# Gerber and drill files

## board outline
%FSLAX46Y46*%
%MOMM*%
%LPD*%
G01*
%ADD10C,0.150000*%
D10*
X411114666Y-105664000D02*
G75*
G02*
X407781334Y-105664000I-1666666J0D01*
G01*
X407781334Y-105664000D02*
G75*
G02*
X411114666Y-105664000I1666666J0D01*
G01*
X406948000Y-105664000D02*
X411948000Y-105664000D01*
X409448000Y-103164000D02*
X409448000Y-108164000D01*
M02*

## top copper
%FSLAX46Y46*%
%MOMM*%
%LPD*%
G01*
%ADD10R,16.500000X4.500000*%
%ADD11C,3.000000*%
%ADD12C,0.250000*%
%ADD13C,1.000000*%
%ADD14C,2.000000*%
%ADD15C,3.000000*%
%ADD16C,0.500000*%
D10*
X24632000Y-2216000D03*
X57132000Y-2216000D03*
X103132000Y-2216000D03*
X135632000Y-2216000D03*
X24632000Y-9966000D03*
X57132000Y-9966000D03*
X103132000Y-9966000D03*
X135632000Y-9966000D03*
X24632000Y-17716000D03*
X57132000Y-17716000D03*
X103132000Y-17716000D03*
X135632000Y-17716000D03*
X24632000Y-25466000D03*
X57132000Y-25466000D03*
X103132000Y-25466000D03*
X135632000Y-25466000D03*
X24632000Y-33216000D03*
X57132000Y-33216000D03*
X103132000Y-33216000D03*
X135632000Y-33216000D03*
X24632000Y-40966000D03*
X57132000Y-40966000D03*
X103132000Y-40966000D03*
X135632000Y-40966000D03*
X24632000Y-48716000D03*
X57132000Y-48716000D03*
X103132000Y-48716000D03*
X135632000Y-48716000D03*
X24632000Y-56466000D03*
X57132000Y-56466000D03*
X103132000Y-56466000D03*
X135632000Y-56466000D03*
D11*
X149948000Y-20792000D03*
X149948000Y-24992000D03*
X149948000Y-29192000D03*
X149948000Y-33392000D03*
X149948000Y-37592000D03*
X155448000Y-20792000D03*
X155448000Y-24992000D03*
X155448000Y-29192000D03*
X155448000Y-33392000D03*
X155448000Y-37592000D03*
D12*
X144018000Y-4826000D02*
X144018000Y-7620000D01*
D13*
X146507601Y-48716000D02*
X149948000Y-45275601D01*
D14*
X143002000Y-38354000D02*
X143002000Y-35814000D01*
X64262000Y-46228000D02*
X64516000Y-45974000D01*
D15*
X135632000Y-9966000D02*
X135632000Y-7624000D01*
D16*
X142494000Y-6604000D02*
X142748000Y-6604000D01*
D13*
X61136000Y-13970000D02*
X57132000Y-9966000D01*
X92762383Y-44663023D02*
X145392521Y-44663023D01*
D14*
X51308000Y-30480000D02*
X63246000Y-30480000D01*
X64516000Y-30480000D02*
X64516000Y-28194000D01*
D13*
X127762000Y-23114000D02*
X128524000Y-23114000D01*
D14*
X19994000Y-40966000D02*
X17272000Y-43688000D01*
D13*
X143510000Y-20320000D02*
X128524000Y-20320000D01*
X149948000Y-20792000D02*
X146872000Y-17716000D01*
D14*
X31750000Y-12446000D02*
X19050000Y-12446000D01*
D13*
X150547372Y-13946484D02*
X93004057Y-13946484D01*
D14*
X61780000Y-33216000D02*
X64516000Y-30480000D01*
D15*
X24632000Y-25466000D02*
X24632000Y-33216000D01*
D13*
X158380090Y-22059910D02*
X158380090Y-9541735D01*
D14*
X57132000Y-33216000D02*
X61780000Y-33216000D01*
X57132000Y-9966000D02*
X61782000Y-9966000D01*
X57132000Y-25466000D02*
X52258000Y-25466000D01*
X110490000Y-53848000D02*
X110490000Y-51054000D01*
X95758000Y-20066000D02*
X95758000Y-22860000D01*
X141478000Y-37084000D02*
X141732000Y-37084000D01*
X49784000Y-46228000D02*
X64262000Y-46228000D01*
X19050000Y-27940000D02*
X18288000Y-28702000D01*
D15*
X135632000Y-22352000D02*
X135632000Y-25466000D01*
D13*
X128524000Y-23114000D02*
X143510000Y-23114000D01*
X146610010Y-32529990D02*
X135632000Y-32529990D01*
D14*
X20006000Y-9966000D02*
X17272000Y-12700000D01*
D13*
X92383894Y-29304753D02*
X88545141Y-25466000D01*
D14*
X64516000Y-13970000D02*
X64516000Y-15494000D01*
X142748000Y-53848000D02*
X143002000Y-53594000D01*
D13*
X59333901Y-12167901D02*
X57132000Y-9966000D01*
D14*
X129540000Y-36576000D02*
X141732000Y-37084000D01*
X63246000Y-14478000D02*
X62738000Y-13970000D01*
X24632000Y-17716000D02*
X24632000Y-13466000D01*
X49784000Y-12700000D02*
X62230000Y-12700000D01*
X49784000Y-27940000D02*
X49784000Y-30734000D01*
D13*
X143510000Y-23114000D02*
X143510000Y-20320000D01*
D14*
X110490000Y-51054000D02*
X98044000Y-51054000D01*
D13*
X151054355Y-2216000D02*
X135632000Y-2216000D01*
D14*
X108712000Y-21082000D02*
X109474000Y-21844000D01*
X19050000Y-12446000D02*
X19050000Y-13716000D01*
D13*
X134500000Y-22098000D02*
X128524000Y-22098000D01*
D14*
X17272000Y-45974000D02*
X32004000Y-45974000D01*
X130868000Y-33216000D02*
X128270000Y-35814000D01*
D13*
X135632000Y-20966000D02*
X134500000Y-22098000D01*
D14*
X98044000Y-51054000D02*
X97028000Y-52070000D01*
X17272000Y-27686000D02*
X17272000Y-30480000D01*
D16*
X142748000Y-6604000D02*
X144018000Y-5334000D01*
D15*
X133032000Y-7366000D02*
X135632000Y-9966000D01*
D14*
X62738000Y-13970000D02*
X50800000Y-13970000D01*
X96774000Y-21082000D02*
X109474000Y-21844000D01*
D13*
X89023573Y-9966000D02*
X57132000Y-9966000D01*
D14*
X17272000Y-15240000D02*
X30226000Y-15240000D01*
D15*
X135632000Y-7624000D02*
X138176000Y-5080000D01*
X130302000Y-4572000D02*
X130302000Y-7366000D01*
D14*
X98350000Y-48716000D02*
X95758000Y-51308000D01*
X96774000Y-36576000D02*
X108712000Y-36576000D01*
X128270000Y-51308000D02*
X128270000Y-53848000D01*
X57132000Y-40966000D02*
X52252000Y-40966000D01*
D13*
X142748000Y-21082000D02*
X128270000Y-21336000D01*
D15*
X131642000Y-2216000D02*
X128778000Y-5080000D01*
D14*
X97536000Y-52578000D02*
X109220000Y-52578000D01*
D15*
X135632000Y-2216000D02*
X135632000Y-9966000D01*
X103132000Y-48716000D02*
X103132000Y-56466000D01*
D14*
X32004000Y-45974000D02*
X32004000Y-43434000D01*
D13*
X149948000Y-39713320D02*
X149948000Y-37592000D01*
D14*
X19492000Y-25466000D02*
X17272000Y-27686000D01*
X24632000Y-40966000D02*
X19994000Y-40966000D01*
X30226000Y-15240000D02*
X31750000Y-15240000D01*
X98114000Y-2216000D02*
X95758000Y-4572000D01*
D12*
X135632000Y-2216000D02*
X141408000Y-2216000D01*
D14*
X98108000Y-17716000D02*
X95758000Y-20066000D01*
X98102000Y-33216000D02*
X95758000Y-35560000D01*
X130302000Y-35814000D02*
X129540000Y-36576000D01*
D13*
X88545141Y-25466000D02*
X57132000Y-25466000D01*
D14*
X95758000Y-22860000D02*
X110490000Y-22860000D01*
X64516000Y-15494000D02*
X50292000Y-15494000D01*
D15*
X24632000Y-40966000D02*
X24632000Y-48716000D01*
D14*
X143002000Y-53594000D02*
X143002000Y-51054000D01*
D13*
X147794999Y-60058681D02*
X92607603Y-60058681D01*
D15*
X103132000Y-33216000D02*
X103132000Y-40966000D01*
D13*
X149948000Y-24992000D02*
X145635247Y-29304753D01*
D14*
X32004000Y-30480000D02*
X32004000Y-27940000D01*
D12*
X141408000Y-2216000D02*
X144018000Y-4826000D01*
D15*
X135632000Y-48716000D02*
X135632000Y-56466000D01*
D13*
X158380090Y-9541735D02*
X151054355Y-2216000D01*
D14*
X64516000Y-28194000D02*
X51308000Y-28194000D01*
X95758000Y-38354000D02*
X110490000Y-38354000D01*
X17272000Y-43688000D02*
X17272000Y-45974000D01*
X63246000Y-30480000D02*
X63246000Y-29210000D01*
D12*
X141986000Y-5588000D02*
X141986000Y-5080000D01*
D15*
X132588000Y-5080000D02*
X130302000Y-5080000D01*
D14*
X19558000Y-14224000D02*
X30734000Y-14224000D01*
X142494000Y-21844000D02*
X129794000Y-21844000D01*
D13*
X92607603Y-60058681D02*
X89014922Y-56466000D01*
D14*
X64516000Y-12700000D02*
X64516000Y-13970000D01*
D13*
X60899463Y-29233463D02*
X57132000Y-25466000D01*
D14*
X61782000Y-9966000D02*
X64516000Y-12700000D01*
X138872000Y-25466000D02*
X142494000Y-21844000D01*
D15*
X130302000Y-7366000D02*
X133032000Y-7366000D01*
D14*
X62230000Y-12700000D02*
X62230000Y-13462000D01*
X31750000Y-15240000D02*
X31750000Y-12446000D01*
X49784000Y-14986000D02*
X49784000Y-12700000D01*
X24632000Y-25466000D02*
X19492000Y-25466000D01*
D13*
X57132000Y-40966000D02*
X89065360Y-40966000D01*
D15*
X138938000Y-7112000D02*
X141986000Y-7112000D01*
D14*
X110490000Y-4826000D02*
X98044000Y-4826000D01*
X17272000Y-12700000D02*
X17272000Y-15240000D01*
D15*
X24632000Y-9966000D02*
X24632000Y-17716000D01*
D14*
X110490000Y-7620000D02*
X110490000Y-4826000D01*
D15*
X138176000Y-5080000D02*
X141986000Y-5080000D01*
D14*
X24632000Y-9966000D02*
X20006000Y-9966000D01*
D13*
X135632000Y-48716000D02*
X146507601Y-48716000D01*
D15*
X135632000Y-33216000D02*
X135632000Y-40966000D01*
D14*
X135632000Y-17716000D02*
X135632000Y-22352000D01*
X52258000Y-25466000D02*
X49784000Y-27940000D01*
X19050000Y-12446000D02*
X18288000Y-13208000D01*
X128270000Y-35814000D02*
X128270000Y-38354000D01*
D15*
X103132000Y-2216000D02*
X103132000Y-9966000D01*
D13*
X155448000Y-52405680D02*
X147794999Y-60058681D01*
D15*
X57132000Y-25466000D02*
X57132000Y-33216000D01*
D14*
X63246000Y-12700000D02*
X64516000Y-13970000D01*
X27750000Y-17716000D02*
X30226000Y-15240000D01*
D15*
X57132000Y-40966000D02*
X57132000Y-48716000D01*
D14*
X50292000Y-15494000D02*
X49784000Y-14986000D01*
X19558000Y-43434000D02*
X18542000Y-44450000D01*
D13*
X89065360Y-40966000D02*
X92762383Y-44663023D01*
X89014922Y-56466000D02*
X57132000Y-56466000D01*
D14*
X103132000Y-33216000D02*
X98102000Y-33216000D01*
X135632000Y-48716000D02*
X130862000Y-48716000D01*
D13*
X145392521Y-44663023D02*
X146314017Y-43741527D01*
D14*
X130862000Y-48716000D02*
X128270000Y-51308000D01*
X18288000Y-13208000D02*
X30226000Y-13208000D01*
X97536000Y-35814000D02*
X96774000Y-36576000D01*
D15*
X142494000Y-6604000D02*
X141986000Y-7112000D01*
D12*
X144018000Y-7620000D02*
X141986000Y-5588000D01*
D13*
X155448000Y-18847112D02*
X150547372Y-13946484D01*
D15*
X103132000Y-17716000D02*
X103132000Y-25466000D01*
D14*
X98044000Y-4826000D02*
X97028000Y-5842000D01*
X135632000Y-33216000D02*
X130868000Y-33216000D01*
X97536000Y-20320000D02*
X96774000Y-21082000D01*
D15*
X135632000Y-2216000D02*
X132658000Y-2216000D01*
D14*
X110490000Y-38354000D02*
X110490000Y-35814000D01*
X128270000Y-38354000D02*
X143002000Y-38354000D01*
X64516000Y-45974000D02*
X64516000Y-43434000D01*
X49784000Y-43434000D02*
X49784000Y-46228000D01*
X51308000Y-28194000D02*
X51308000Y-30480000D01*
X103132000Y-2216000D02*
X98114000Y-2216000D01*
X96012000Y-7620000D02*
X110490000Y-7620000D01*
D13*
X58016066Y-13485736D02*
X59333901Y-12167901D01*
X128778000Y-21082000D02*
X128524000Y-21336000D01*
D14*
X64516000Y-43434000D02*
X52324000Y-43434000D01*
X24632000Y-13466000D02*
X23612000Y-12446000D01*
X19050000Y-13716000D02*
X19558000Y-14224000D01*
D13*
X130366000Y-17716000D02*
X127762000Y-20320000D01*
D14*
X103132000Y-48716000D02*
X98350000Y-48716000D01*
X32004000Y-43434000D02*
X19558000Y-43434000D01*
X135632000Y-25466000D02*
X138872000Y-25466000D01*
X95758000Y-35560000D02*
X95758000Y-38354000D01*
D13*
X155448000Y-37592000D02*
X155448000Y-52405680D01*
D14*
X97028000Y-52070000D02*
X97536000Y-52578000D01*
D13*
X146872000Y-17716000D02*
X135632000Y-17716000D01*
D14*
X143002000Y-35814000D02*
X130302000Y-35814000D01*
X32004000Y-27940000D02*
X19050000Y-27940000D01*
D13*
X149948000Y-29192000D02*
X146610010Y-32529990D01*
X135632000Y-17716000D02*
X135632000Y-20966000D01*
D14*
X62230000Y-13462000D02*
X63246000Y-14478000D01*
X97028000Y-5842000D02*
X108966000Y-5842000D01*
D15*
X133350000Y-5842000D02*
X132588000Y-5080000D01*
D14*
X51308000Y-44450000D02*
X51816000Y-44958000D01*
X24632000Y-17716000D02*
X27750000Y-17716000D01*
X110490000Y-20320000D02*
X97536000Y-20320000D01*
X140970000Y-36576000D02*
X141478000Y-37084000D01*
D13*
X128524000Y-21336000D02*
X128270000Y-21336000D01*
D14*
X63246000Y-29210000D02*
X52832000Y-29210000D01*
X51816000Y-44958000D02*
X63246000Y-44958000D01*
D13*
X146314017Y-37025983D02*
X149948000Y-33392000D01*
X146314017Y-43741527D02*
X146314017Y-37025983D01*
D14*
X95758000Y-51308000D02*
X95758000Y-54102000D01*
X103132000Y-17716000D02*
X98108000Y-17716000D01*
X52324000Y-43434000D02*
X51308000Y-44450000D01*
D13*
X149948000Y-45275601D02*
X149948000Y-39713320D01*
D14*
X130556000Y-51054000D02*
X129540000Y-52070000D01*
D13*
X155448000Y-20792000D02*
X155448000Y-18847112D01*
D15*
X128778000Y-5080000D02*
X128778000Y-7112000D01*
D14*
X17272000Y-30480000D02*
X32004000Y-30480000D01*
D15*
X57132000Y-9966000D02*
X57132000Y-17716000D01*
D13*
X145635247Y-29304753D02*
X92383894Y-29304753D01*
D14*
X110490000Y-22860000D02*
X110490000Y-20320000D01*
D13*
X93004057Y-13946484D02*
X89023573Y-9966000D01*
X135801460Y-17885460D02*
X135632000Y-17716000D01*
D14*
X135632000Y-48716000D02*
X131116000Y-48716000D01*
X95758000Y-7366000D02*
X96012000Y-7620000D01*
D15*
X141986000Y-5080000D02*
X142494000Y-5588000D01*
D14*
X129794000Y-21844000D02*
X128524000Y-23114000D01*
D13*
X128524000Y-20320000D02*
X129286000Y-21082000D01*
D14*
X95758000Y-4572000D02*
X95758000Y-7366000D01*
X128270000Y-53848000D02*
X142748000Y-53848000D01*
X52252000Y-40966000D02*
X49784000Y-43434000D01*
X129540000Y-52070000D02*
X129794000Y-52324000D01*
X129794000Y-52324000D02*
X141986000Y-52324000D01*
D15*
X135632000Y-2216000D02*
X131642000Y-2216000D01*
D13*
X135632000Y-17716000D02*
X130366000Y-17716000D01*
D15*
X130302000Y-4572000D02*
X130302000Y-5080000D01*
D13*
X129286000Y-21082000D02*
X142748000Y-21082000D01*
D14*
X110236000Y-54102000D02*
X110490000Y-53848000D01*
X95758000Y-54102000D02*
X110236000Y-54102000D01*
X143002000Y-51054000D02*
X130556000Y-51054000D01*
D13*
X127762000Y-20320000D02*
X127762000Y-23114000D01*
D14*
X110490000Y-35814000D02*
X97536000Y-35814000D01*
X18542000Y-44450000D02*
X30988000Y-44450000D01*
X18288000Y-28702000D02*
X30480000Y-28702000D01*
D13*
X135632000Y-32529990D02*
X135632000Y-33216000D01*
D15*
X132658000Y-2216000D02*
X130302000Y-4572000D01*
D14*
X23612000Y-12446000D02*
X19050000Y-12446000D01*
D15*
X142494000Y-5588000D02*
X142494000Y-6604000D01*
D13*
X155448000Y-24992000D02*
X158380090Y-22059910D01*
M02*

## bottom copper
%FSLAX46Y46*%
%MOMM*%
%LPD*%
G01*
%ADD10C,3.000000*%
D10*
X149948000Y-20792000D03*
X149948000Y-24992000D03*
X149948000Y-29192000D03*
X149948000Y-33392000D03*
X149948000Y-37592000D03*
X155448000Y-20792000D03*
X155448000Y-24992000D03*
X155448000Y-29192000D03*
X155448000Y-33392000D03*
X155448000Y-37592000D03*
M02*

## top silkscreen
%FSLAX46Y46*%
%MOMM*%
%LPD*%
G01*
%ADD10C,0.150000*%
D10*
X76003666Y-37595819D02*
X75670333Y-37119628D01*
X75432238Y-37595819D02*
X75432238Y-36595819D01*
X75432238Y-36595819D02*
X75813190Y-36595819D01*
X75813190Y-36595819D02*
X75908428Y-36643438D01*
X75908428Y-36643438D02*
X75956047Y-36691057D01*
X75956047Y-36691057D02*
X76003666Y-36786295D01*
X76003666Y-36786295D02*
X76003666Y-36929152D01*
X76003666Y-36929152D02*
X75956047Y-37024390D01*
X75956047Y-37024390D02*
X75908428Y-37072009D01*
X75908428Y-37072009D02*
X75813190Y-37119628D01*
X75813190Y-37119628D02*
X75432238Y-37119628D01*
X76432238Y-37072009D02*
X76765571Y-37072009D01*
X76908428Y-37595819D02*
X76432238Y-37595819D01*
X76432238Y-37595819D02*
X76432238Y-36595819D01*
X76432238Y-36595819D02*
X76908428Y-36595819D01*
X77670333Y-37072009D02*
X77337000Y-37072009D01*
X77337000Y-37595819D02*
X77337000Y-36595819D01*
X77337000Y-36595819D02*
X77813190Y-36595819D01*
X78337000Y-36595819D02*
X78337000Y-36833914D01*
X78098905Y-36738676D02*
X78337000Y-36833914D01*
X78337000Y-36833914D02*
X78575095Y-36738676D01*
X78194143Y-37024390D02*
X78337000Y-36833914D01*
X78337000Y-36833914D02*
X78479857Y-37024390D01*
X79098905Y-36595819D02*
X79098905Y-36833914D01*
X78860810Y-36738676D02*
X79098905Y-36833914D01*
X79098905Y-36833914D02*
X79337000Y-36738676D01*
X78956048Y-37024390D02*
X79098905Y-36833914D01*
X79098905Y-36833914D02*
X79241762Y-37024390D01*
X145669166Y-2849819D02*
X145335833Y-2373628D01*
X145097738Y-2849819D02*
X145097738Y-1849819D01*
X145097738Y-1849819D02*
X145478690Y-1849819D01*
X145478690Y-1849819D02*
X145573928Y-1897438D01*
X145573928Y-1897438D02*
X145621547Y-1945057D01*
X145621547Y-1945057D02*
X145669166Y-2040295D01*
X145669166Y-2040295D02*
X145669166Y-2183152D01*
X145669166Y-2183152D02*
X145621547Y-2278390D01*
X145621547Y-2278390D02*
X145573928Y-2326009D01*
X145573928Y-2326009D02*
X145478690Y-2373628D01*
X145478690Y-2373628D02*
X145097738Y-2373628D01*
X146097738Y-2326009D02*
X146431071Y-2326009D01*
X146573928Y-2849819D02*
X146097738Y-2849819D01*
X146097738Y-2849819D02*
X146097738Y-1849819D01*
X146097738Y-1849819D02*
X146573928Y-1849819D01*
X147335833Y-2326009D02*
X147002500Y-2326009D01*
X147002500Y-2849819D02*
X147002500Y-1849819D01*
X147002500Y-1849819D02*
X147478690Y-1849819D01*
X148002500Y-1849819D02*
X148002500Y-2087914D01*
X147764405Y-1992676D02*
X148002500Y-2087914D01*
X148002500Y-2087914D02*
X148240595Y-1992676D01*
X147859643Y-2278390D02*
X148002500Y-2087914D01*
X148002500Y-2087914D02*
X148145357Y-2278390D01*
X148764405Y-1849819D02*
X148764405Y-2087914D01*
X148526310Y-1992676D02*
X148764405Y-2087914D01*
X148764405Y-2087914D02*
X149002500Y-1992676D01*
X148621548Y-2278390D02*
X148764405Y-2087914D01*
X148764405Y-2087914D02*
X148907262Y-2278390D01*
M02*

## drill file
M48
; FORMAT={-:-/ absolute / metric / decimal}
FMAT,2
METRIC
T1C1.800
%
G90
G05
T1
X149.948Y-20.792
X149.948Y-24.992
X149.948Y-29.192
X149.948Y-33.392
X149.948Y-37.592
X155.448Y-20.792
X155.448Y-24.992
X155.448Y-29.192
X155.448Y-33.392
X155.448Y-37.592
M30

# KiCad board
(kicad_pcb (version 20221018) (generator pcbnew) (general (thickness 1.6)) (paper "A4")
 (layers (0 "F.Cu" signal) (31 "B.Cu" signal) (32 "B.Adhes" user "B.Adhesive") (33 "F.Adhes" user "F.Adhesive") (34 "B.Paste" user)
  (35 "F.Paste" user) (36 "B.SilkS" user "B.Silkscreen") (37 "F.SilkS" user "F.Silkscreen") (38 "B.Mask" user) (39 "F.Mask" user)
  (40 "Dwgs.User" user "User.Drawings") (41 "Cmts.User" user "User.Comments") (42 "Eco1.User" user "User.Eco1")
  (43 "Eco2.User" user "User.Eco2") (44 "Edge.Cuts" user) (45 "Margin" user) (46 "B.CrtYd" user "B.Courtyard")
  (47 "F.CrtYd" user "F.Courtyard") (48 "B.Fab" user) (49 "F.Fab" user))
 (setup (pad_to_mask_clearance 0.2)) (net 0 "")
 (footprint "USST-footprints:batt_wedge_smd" (layer "F.Cu") (at 77.337 37.141)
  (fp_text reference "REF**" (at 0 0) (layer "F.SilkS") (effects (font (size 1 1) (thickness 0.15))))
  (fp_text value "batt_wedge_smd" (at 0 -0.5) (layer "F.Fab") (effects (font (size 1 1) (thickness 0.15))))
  (pad "1" smd rect (at -52.705 -34.925 90) (size 4.5 16.5) (layers "F.Cu" "F.Paste" "F.Mask"))
  (pad "1" smd rect (at -20.205 -34.925 90) (size 4.5 16.5) (layers "F.Cu" "F.Paste" "F.Mask"))
  (pad "1" smd rect (at 25.795 -34.925 90) (size 4.5 16.5) (layers "F.Cu" "F.Paste" "F.Mask"))
  (pad "1" smd rect (at 58.295 -34.925 90) (size 4.5 16.5) (layers "F.Cu" "F.Paste" "F.Mask"))
  (pad "2" smd rect (at -52.705 -27.175 90) (size 4.5 16.5) (layers "F.Cu" "F.Paste" "F.Mask"))
  (pad "2" smd rect (at -20.205 -27.175 90) (size 4.5 16.5) (layers "F.Cu" "F.Paste" "F.Mask"))
  (pad "2" smd rect (at 25.795 -27.175 90) (size 4.5 16.5) (layers "F.Cu" "F.Paste" "F.Mask"))
  (pad "2" smd rect (at 58.295 -27.175 90) (size 4.5 16.5) (layers "F.Cu" "F.Paste" "F.Mask"))
  (pad "3" smd rect (at -52.705 -19.425 90) (size 4.5 16.5) (layers "F.Cu" "F.Paste" "F.Mask"))
  (pad "3" smd rect (at -20.205 -19.425 90) (size 4.5 16.5) (layers "F.Cu" "F.Paste" "F.Mask"))
  (pad "3" smd rect (at 25.795 -19.425 90) (size 4.5 16.5) (layers "F.Cu" "F.Paste" "F.Mask"))
  (pad "3" smd rect (at 58.295 -19.425 90) (size 4.5 16.5) (layers "F.Cu" "F.Paste" "F.Mask"))
  (pad "4" smd rect (at -52.705 -11.675 90) (size 4.5 16.5) (layers "F.Cu" "F.Paste" "F.Mask"))
  (pad "4" smd rect (at -20.205 -11.675 90) (size 4.5 16.5) (layers "F.Cu" "F.Paste" "F.Mask"))
  (pad "4" smd rect (at 25.795 -11.675 90) (size 4.5 16.5) (layers "F.Cu" "F.Paste" "F.Mask"))
  (pad "4" smd rect (at 58.295 -11.675 90) (size 4.5 16.5) (layers "F.Cu" "F.Paste" "F.Mask"))
  (pad "5" smd rect (at -52.705 -3.925 90) (size 4.5 16.5) (layers "F.Cu" "F.Paste" "F.Mask"))
  (pad "5" smd rect (at -20.205 -3.925 90) (size 4.5 16.5) (layers "F.Cu" "F.Paste" "F.Mask"))
  (pad "5" smd rect (at 25.795 -3.925 90) (size 4.5 16.5) (layers "F.Cu" "F.Paste" "F.Mask"))
  (pad "5" smd rect (at 58.295 -3.925 90) (size 4.5 16.5) (layers "F.Cu" "F.Paste" "F.Mask"))
  (pad "6" smd rect (at -52.705 3.825 90) (size 4.5 16.5) (layers "F.Cu" "F.Paste" "F.Mask"))
  (pad "6" smd rect (at -20.205 3.825 90) (size 4.5 16.5) (layers "F.Cu" "F.Paste" "F.Mask"))
  (pad "6" smd rect (at 25.795 3.825 90) (size 4.5 16.5) (layers "F.Cu" "F.Paste" "F.Mask"))
  (pad "6" smd rect (at 58.295 3.825 90) (size 4.5 16.5) (layers "F.Cu" "F.Paste" "F.Mask"))
  (pad "7" smd rect (at -52.705 11.575 90) (size 4.5 16.5) (layers "F.Cu" "F.Paste" "F.Mask"))
  (pad "7" smd rect (at -20.205 11.575 90) (size 4.5 16.5) (layers "F.Cu" "F.Paste" "F.Mask"))
  (pad "7" smd rect (at 25.795 11.575 90) (size 4.5 16.5) (layers "F.Cu" "F.Paste" "F.Mask"))
  (pad "7" smd rect (at 58.295 11.575 90) (size 4.5 16.5) (layers "F.Cu" "F.Paste" "F.Mask"))
  (pad "8" smd rect (at -52.705 19.325 90) (size 4.5 16.5) (layers "F.Cu" "F.Paste" "F.Mask"))
  (pad "8" smd rect (at -20.205 19.325 90) (size 4.5 16.5) (layers "F.Cu" "F.Paste" "F.Mask"))
  (pad "8" smd rect (at 25.795 19.325 90) (size 4.5 16.5) (layers "F.Cu" "F.Paste" "F.Mask"))
  (pad "8" smd rect (at 58.295 19.325 90) (size 4.5 16.5) (layers "F.Cu" "F.Paste" "F.Mask")))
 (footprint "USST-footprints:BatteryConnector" (layer "F.Cu") (at 149.948 37.592)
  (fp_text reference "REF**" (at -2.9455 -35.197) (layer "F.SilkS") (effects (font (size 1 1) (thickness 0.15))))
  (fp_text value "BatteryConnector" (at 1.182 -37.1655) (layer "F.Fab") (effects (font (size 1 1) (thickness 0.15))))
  (pad "" np_thru_hole circle (at 0 -16.8) (size 3 3) (drill 1.8) (layers "*.Cu"))
  (pad "" np_thru_hole circle (at 0 -12.6) (size 3 3) (drill 1.8) (layers "*.Cu"))
  (pad "" np_thru_hole circle (at 0 -8.4) (size 3 3) (drill 1.8) (layers "*.Cu"))
  (pad "" np_thru_hole circle (at 0 -4.2) (size 3 3) (drill 1.8) (layers "*.Cu"))
  (pad "" np_thru_hole circle (at 0 0) (size 3 3) (drill 1.8) (layers "*.Cu"))
  (pad "" np_thru_hole circle (at 5.5 -16.8) (size 3 3) (drill 1.8) (layers "*.Cu"))
  (pad "" np_thru_hole circle (at 5.5 -12.6) (size 3 3) (drill 1.8) (layers "*.Cu"))
  (pad "" np_thru_hole circle (at 5.5 -8.4) (size 3 3) (drill 1.8) (layers "*.Cu"))
  (pad "" np_thru_hole circle (at 5.5 -4.2) (size 3 3) (drill 1.8) (layers "*.Cu"))
  (pad "" np_thru_hole circle (at 5.5 0) (size 3 3) (drill 1.8) (layers "*.Cu")))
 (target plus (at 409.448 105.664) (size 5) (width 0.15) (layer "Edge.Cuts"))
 (segment (start 144.018 4.826) (end 144.018 7.62) (width 0.25) (layer "F.Cu") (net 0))
 (segment (start 146.507601 48.716) (end 149.948 45.275601) (width 1) (layer "F.Cu") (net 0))
 (segment (start 143.002 38.354) (end 143.002 35.814) (width 2) (layer "F.Cu") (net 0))
 (segment (start 64.262 46.228) (end 64.516 45.974) (width 2) (layer "F.Cu") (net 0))
 (segment (start 135.632 9.966) (end 135.632 7.624) (width 3) (layer "F.Cu") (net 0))
 (segment (start 142.494 6.604) (end 142.748 6.604) (width 0.5) (layer "F.Cu") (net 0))
 (segment (start 61.136 13.97) (end 57.132 9.966) (width 1) (layer "F.Cu") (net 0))
 (segment (start 92.762383 44.663023) (end 145.392521 44.663023) (width 1) (layer "F.Cu") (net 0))
 (segment (start 51.308 30.48) (end 63.246 30.48) (width 2) (layer "F.Cu") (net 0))
 (segment (start 64.516 30.48) (end 64.516 28.194) (width 2) (layer "F.Cu") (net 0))
 (segment (start 127.762 23.114) (end 128.524 23.114) (width 1) (layer "F.Cu") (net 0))
 (segment (start 19.994 40.966) (end 17.272 43.688) (width 2) (layer "F.Cu") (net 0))
 (segment (start 143.51 20.32) (end 128.524 20.32) (width 1) (layer "F.Cu") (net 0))
 (segment (start 149.948 20.792) (end 146.872 17.716) (width 1) (layer "F.Cu") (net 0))
 (segment (start 31.75 12.446) (end 19.05 12.446) (width 2) (layer "F.Cu") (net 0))
 (segment (start 150.547372 13.946484) (end 93.004057 13.946484) (width 1) (layer "F.Cu") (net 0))
 (segment (start 61.78 33.216) (end 64.516 30.48) (width 2) (layer "F.Cu") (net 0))
 (segment (start 24.632 25.466) (end 24.632 33.216) (width 3) (layer "F.Cu") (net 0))
 (segment (start 158.38009 22.05991) (end 158.38009 9.541735) (width 1) (layer "F.Cu") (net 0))
 (segment (start 57.132 33.216) (end 61.78 33.216) (width 2) (layer "F.Cu") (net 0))
 (segment (start 57.132 9.966) (end 61.782 9.966) (width 2) (layer "F.Cu") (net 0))
 (segment (start 57.132 25.466) (end 52.258 25.466) (width 2) (layer "F.Cu") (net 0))
 (segment (start 110.49 53.848) (end 110.49 51.054) (width 2) (layer "F.Cu") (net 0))
 (segment (start 95.758 20.066) (end 95.758 22.86) (width 2) (layer "F.Cu") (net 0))
 (segment (start 141.478 37.084) (end 141.732 37.084) (width 2) (layer "F.Cu") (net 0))
 (segment (start 49.784 46.228) (end 64.262 46.228) (width 2) (layer "F.Cu") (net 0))
 (segment (start 19.05 27.94) (end 18.288 28.702) (width 2) (layer "F.Cu") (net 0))
 (segment (start 135.632 22.352) (end 135.632 25.466) (width 3) (layer "F.Cu") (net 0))
 (segment (start 128.524 23.114) (end 143.51 23.114) (width 1) (layer "F.Cu") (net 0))
 (segment (start 146.61001 32.52999) (end 135.632 32.52999) (width 1) (layer "F.Cu") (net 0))
 (segment (start 20.006 9.966) (end 17.272 12.7) (width 2) (layer "F.Cu") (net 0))
 (segment (start 92.383894 29.304753) (end 88.545141 25.466) (width 1) (layer "F.Cu") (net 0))
 (segment (start 64.516 13.97) (end 64.516 15.494) (width 2) (layer "F.Cu") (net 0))
 (segment (start 142.748 53.848) (end 143.002 53.594) (width 2) (layer "F.Cu") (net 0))
 (segment (start 59.333901 12.167901) (end 57.132 9.966) (width 1) (layer "F.Cu") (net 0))
 (segment (start 129.54 36.576) (end 141.732 37.084) (width 2) (layer "F.Cu") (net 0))
 (segment (start 63.246 14.478) (end 62.738 13.97) (width 2) (layer "F.Cu") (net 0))
 (segment (start 24.632 17.716) (end 24.632 13.466) (width 2) (layer "F.Cu") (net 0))
 (segment (start 49.784 12.7) (end 62.23 12.7) (width 2) (layer "F.Cu") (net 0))
 (segment (start 49.784 27.94) (end 49.784 30.734) (width 2) (layer "F.Cu") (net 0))
 (segment (start 143.51 23.114) (end 143.51 20.32) (width 1) (layer "F.Cu") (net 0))
 (segment (start 110.49 51.054) (end 98.044 51.054) (width 2) (layer "F.Cu") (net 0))
 (segment (start 151.054355 2.216) (end 135.632 2.216) (width 1) (layer "F.Cu") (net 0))
 (segment (start 108.712 21.082) (end 109.474 21.844) (width 2) (layer "F.Cu") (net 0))
 (segment (start 19.05 12.446) (end 19.05 13.716) (width 2) (layer "F.Cu") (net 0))
 (segment (start 134.5 22.098) (end 128.524 22.098) (width 1) (layer "F.Cu") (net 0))
 (segment (start 17.272 45.974) (end 32.004 45.974) (width 2) (layer "F.Cu") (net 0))
 (segment (start 130.868 33.216) (end 128.27 35.814) (width 2) (layer "F.Cu") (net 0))
 (segment (start 135.632 20.966) (end 134.5 22.098) (width 1) (layer "F.Cu") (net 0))
 (segment (start 98.044 51.054) (end 97.028 52.07) (width 2) (layer "F.Cu") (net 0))
 (segment (start 17.272 27.686) (end 17.272 30.48) (width 2) (layer "F.Cu") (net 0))
 (segment (start 142.748 6.604) (end 144.018 5.334) (width 0.5) (layer "F.Cu") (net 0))
 (segment (start 133.032 7.366) (end 135.632 9.966) (width 3) (layer "F.Cu") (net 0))
 (segment (start 62.738 13.97) (end 50.8 13.97) (width 2) (layer "F.Cu") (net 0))
 (segment (start 96.774 21.082) (end 109.474 21.844) (width 2) (layer "F.Cu") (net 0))
 (segment (start 89.023573 9.966) (end 57.132 9.966) (width 1) (layer "F.Cu") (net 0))
 (segment (start 17.272 15.24) (end 30.226 15.24) (width 2) (layer "F.Cu") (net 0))
 (segment (start 135.632 7.624) (end 138.176 5.08) (width 3) (layer "F.Cu") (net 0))
 (segment (start 130.302 4.572) (end 130.302 7.366) (width 3) (layer "F.Cu") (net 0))
 (segment (start 98.35 48.716) (end 95.758 51.308) (width 2) (layer "F.Cu") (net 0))
 (segment (start 96.774 36.576) (end 108.712 36.576) (width 2) (layer "F.Cu") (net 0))
 (segment (start 128.27 51.308) (end 128.27 53.848) (width 2) (layer "F.Cu") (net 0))
 (segment (start 57.132 40.966) (end 52.252 40.966) (width 2) (layer "F.Cu") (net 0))
 (segment (start 142.748 21.082) (end 128.27 21.336) (width 1) (layer "F.Cu") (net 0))
 (segment (start 131.642 2.216) (end 128.778 5.08) (width 3) (layer "F.Cu") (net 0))
 (segment (start 97.536 52.578) (end 109.22 52.578) (width 2) (layer "F.Cu") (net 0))
 (segment (start 135.632 2.216) (end 135.632 9.966) (width 3) (layer "F.Cu") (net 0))
 (segment (start 103.132 48.716) (end 103.132 56.466) (width 3) (layer "F.Cu") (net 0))
 (segment (start 32.004 45.974) (end 32.004 43.434) (width 2) (layer "F.Cu") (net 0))
 (segment (start 149.948 39.71332) (end 149.948 37.592) (width 1) (layer "F.Cu") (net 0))
 (segment (start 19.492 25.466) (end 17.272 27.686) (width 2) (layer "F.Cu") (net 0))
 (segment (start 24.632 40.966) (end 19.994 40.966) (width 2) (layer "F.Cu") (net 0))
 (segment (start 30.226 15.24) (end 31.75 15.24) (width 2) (layer "F.Cu") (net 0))
 (segment (start 98.114 2.216) (end 95.758 4.572) (width 2) (layer "F.Cu") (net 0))
 (segment (start 135.632 2.216) (end 141.408 2.216) (width 0.25) (layer "F.Cu") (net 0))
 (segment (start 98.108 17.716) (end 95.758 20.066) (width 2) (layer "F.Cu") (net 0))
 (segment (start 98.102 33.216) (end 95.758 35.56) (width 2) (layer "F.Cu") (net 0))
 (segment (start 130.302 35.814) (end 129.54 36.576) (width 2) (layer "F.Cu") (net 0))
 (segment (start 88.545141 25.466) (end 57.132 25.466) (width 1) (layer "F.Cu") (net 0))
 (segment (start 95.758 22.86) (end 110.49 22.86) (width 2) (layer "F.Cu") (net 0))
 (segment (start 64.516 15.494) (end 50.292 15.494) (width 2) (layer "F.Cu") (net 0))
 (segment (start 24.632 40.966) (end 24.632 48.716) (width 3) (layer "F.Cu") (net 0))
 (segment (start 143.002 53.594) (end 143.002 51.054) (width 2) (layer "F.Cu") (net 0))
 (segment (start 147.794999 60.058681) (end 92.607603 60.058681) (width 1) (layer "F.Cu") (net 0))
 (segment (start 103.132 33.216) (end 103.132 40.966) (width 3) (layer "F.Cu") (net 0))
 (segment (start 149.948 24.992) (end 145.635247 29.304753) (width 1) (layer "F.Cu") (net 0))
 (segment (start 32.004 30.48) (end 32.004 27.94) (width 2) (layer "F.Cu") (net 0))
 (segment (start 141.408 2.216) (end 144.018 4.826) (width 0.25) (layer "F.Cu") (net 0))
 (segment (start 135.632 48.716) (end 135.632 56.466) (width 3) (layer "F.Cu") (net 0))
 (segment (start 158.38009 9.541735) (end 151.054355 2.216) (width 1) (layer "F.Cu") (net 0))
 (segment (start 64.516 28.194) (end 51.308 28.194) (width 2) (layer "F.Cu") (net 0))
 (segment (start 95.758 38.354) (end 110.49 38.354) (width 2) (layer "F.Cu") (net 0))
 (segment (start 17.272 43.688) (end 17.272 45.974) (width 2) (layer "F.Cu") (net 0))
 (segment (start 63.246 30.48) (end 63.246 29.21) (width 2) (layer "F.Cu") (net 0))
 (segment (start 141.986 5.588) (end 141.986 5.08) (width 0.25) (layer "F.Cu") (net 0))
 (segment (start 132.588 5.08) (end 130.302 5.08) (width 3) (layer "F.Cu") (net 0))
 (segment (start 19.558 14.224) (end 30.734 14.224) (width 2) (layer "F.Cu") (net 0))
 (segment (start 142.494 21.844) (end 129.794 21.844) (width 2) (layer "F.Cu") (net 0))
 (segment (start 92.607603 60.058681) (end 89.014922 56.466) (width 1) (layer "F.Cu") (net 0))
 (segment (start 64.516 12.7) (end 64.516 13.97) (width 2) (layer "F.Cu") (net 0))
 (segment (start 60.899463 29.233463) (end 57.132 25.466) (width 1) (layer "F.Cu") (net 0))
 (segment (start 61.782 9.966) (end 64.516 12.7) (width 2) (layer "F.Cu") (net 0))
 (segment (start 138.872 25.466) (end 142.494 21.844) (width 2) (layer "F.Cu") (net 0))
 (segment (start 130.302 7.366) (end 133.032 7.366) (width 3) (layer "F.Cu") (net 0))
 (segment (start 62.23 12.7) (end 62.23 13.462) (width 2) (layer "F.Cu") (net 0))
 (segment (start 31.75 15.24) (end 31.75 12.446) (width 2) (layer "F.Cu") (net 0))
 (segment (start 49.784 14.986) (end 49.784 12.7) (width 2) (layer "F.Cu") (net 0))
 (segment (start 24.632 25.466) (end 19.492 25.466) (width 2) (layer "F.Cu") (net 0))
 (segment (start 57.132 40.966) (end 89.06536 40.966) (width 1) (layer "F.Cu") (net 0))
 (segment (start 138.938 7.112) (end 141.986 7.112) (width 3) (layer "F.Cu") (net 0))
 (segment (start 110.49 4.826) (end 98.044 4.826) (width 2) (layer "F.Cu") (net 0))
 (segment (start 17.272 12.7) (end 17.272 15.24) (width 2) (layer "F.Cu") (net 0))
 (segment (start 24.632 9.966) (end 24.632 17.716) (width 3) (layer "F.Cu") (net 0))
 (segment (start 110.49 7.62) (end 110.49 4.826) (width 2) (layer "F.Cu") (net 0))
 (segment (start 138.176 5.08) (end 141.986 5.08) (width 3) (layer "F.Cu") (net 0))
 (segment (start 24.632 9.966) (end 20.006 9.966) (width 2) (layer "F.Cu") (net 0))
 (segment (start 135.632 48.716) (end 146.507601 48.716) (width 1) (layer "F.Cu") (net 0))
 (segment (start 135.632 33.216) (end 135.632 40.966) (width 3) (layer "F.Cu") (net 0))
 (segment (start 135.632 17.716) (end 135.632 22.352) (width 2) (layer "F.Cu") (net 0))
 (segment (start 52.258 25.466) (end 49.784 27.94) (width 2) (layer "F.Cu") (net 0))
 (segment (start 19.05 12.446) (end 18.288 13.208) (width 2) (layer "F.Cu") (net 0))
 (segment (start 128.27 35.814) (end 128.27 38.354) (width 2) (layer "F.Cu") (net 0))
 (segment (start 103.132 2.216) (end 103.132 9.966) (width 3) (layer "F.Cu") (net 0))
 (segment (start 155.448 52.40568) (end 147.794999 60.058681) (width 1) (layer "F.Cu") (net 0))
 (segment (start 57.132 25.466) (end 57.132 33.216) (width 3) (layer "F.Cu") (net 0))
 (segment (start 63.246 12.7) (end 64.516 13.97) (width 2) (layer "F.Cu") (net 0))
 (segment (start 27.75 17.716) (end 30.226 15.24) (width 2) (layer "F.Cu") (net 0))
 (segment (start 57.132 40.966) (end 57.132 48.716) (width 3) (layer "F.Cu") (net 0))
 (segment (start 50.292 15.494) (end 49.784 14.986) (width 2) (layer "F.Cu") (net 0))
 (segment (start 19.558 43.434) (end 18.542 44.45) (width 2) (layer "F.Cu") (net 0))
 (segment (start 89.06536 40.966) (end 92.762383 44.663023) (width 1) (layer "F.Cu") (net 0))
 (segment (start 89.014922 56.466) (end 57.132 56.466) (width 1) (layer "F.Cu") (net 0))
 (segment (start 103.132 33.216) (end 98.102 33.216) (width 2) (layer "F.Cu") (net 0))
 (segment (start 135.632 48.716) (end 130.862 48.716) (width 2) (layer "F.Cu") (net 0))
 (segment (start 145.392521 44.663023) (end 146.314017 43.741527) (width 1) (layer "F.Cu") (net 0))
 (segment (start 130.862 48.716) (end 128.27 51.308) (width 2) (layer "F.Cu") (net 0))
 (segment (start 18.288 13.208) (end 30.226 13.208) (width 2) (layer "F.Cu") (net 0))
 (segment (start 97.536 35.814) (end 96.774 36.576) (width 2) (layer "F.Cu") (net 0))
 (segment (start 142.494 6.604) (end 141.986 7.112) (width 3) (layer "F.Cu") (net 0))
 (segment (start 144.018 7.62) (end 141.986 5.588) (width 0.25) (layer "F.Cu") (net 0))
 (segment (start 155.448 18.847112) (end 150.547372 13.946484) (width 1) (layer "F.Cu") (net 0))
 (segment (start 103.132 17.716) (end 103.132 25.466) (width 3) (layer "F.Cu") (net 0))
 (segment (start 98.044 4.826) (end 97.028 5.842) (width 2) (layer "F.Cu") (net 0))
 (segment (start 135.632 33.216) (end 130.868 33.216) (width 2) (layer "F.Cu") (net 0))
 (segment (start 97.536 20.32) (end 96.774 21.082) (width 2) (layer "F.Cu") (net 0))
 (segment (start 135.632 2.216) (end 132.658 2.216) (width 3) (layer "F.Cu") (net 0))
 (segment (start 110.49 38.354) (end 110.49 35.814) (width 2) (layer "F.Cu") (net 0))
 (segment (start 128.27 38.354) (end 143.002 38.354) (width 2) (layer "F.Cu") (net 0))
 (segment (start 64.516 45.974) (end 64.516 43.434) (width 2) (layer "F.Cu") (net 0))
 (segment (start 49.784 43.434) (end 49.784 46.228) (width 2) (layer "F.Cu") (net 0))
 (segment (start 51.308 28.194) (end 51.308 30.48) (width 2) (layer "F.Cu") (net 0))
 (segment (start 103.132 2.216) (end 98.114 2.216) (width 2) (layer "F.Cu") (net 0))
 (segment (start 96.012 7.62) (end 110.49 7.62) (width 2) (layer "F.Cu") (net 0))
 (segment (start 58.016066 13.485736) (end 59.333901 12.167901) (width 1) (layer "F.Cu") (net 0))
 (segment (start 128.778 21.082) (end 128.524 21.336) (width 1) (layer "F.Cu") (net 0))
 (segment (start 64.516 43.434) (end 52.324 43.434) (width 2) (layer "F.Cu") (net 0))
 (segment (start 24.632 13.466) (end 23.612 12.446) (width 2) (layer "F.Cu") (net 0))
 (segment (start 19.05 13.716) (end 19.558 14.224) (width 2) (layer "F.Cu") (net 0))
 (segment (start 130.366 17.716) (end 127.762 20.32) (width 1) (layer "F.Cu") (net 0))
 (segment (start 103.132 48.716) (end 98.35 48.716) (width 2) (layer "F.Cu") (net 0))
 (segment (start 32.004 43.434) (end 19.558 43.434) (width 2) (layer "F.Cu") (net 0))
 (segment (start 135.632 25.466) (end 138.872 25.466) (width 2) (layer "F.Cu") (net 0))
 (segment (start 95.758 35.56) (end 95.758 38.354) (width 2) (layer "F.Cu") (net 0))
 (segment (start 155.448 37.592) (end 155.448 52.40568) (width 1) (layer "F.Cu") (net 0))
 (segment (start 97.028 52.07) (end 97.536 52.578) (width 2) (layer "F.Cu") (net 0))
 (segment (start 146.872 17.716) (end 135.632 17.716) (width 1) (layer "F.Cu") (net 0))
 (segment (start 143.002 35.814) (end 130.302 35.814) (width 2) (layer "F.Cu") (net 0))
 (segment (start 32.004 27.94) (end 19.05 27.94) (width 2) (layer "F.Cu") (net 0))
 (segment (start 149.948 29.192) (end 146.61001 32.52999) (width 1) (layer "F.Cu") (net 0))
 (segment (start 135.632 17.716) (end 135.632 20.966) (width 1) (layer "F.Cu") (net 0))
 (segment (start 62.23 13.462) (end 63.246 14.478) (width 2) (layer "F.Cu") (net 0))
 (segment (start 97.028 5.842) (end 108.966 5.842) (width 2) (layer "F.Cu") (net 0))
 (segment (start 133.35 5.842) (end 132.588 5.08) (width 3) (layer "F.Cu") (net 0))
 (segment (start 51.308 44.45) (end 51.816 44.958) (width 2) (layer "F.Cu") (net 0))
 (segment (start 24.632 17.716) (end 27.75 17.716) (width 2) (layer "F.Cu") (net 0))
 (segment (start 110.49 20.32) (end 97.536 20.32) (width 2) (layer "F.Cu") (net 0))
 (segment (start 140.97 36.576) (end 141.478 37.084) (width 2) (layer "F.Cu") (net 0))
 (segment (start 128.524 21.336) (end 128.27 21.336) (width 1) (layer "F.Cu") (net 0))
 (segment (start 63.246 29.21) (end 52.832 29.21) (width 2) (layer "F.Cu") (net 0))
 (segment (start 51.816 44.958) (end 63.246 44.958) (width 2) (layer "F.Cu") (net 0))
 (segment (start 146.314017 37.025983) (end 149.948 33.392) (width 1) (layer "F.Cu") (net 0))
 (segment (start 146.314017 43.741527) (end 146.314017 37.025983) (width 1) (layer "F.Cu") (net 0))
 (segment (start 95.758 51.308) (end 95.758 54.102) (width 2) (layer "F.Cu") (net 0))
 (segment (start 103.132 17.716) (end 98.108 17.716) (width 2) (layer "F.Cu") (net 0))
 (segment (start 52.324 43.434) (end 51.308 44.45) (width 2) (layer "F.Cu") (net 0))
 (segment (start 149.948 45.275601) (end 149.948 39.71332) (width 1) (layer "F.Cu") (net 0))
 (segment (start 130.556 51.054) (end 129.54 52.07) (width 2) (layer "F.Cu") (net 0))
 (segment (start 155.448 20.792) (end 155.448 18.847112) (width 1) (layer "F.Cu") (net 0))
 (segment (start 128.778 5.08) (end 128.778 7.112) (width 3) (layer "F.Cu") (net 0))
 (segment (start 17.272 30.48) (end 32.004 30.48) (width 2) (layer "F.Cu") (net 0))
 (segment (start 57.132 9.966) (end 57.132 17.716) (width 3) (layer "F.Cu") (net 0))
 (segment (start 145.635247 29.304753) (end 92.383894 29.304753) (width 1) (layer "F.Cu") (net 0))
 (segment (start 110.49 22.86) (end 110.49 20.32) (width 2) (layer "F.Cu") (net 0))
 (segment (start 93.004057 13.946484) (end 89.023573 9.966) (width 1) (layer "F.Cu") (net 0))
 (segment (start 135.80146 17.88546) (end 135.632 17.716) (width 1) (layer "F.Cu") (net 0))
 (segment (start 135.632 48.716) (end 131.116 48.716) (width 2) (layer "F.Cu") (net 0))
 (segment (start 95.758 7.366) (end 96.012 7.62) (width 2) (layer "F.Cu") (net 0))
 (segment (start 141.986 5.08) (end 142.494 5.588) (width 3) (layer "F.Cu") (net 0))
 (segment (start 129.794 21.844) (end 128.524 23.114) (width 2) (layer "F.Cu") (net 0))
 (segment (start 128.524 20.32) (end 129.286 21.082) (width 1) (layer "F.Cu") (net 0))
 (segment (start 95.758 4.572) (end 95.758 7.366) (width 2) (layer "F.Cu") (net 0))
 (segment (start 128.27 53.848) (end 142.748 53.848) (width 2) (layer "F.Cu") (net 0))
 (segment (start 52.252 40.966) (end 49.784 43.434) (width 2) (layer "F.Cu") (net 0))
 (segment (start 129.54 52.07) (end 129.794 52.324) (width 2) (layer "F.Cu") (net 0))
 (segment (start 129.794 52.324) (end 141.986 52.324) (width 2) (layer "F.Cu") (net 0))
 (segment (start 135.632 2.216) (end 131.642 2.216) (width 3) (layer "F.Cu") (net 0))
 (segment (start 135.632 17.716) (end 130.366 17.716) (width 1) (layer "F.Cu") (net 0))
 (segment (start 130.302 4.572) (end 130.302 5.08) (width 3) (layer "F.Cu") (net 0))
 (segment (start 129.286 21.082) (end 142.748 21.082) (width 1) (layer "F.Cu") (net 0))
 (segment (start 110.236 54.102) (end 110.49 53.848) (width 2) (layer "F.Cu") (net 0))
 (segment (start 95.758 54.102) (end 110.236 54.102) (width 2) (layer "F.Cu") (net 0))
 (segment (start 143.002 51.054) (end 130.556 51.054) (width 2) (layer "F.Cu") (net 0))
 (segment (start 127.762 20.32) (end 127.762 23.114) (width 1) (layer "F.Cu") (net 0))
 (segment (start 110.49 35.814) (end 97.536 35.814) (width 2) (layer "F.Cu") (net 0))
 (segment (start 18.542 44.45) (end 30.988 44.45) (width 2) (layer "F.Cu") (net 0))
 (segment (start 18.288 28.702) (end 30.48 28.702) (width 2) (layer "F.Cu") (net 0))
 (segment (start 135.632 32.52999) (end 135.632 33.216) (width 1) (layer "F.Cu") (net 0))
 (segment (start 132.658 2.216) (end 130.302 4.572) (width 3) (layer "F.Cu") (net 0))
 (segment (start 23.612 12.446) (end 19.05 12.446) (width 2) (layer "F.Cu") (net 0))
 (segment (start 142.494 5.588) (end 142.494 6.604) (width 3) (layer "F.Cu") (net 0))
 (segment (start 155.448 24.992) (end 158.38009 22.05991) (width 1) (layer "F.Cu") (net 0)))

